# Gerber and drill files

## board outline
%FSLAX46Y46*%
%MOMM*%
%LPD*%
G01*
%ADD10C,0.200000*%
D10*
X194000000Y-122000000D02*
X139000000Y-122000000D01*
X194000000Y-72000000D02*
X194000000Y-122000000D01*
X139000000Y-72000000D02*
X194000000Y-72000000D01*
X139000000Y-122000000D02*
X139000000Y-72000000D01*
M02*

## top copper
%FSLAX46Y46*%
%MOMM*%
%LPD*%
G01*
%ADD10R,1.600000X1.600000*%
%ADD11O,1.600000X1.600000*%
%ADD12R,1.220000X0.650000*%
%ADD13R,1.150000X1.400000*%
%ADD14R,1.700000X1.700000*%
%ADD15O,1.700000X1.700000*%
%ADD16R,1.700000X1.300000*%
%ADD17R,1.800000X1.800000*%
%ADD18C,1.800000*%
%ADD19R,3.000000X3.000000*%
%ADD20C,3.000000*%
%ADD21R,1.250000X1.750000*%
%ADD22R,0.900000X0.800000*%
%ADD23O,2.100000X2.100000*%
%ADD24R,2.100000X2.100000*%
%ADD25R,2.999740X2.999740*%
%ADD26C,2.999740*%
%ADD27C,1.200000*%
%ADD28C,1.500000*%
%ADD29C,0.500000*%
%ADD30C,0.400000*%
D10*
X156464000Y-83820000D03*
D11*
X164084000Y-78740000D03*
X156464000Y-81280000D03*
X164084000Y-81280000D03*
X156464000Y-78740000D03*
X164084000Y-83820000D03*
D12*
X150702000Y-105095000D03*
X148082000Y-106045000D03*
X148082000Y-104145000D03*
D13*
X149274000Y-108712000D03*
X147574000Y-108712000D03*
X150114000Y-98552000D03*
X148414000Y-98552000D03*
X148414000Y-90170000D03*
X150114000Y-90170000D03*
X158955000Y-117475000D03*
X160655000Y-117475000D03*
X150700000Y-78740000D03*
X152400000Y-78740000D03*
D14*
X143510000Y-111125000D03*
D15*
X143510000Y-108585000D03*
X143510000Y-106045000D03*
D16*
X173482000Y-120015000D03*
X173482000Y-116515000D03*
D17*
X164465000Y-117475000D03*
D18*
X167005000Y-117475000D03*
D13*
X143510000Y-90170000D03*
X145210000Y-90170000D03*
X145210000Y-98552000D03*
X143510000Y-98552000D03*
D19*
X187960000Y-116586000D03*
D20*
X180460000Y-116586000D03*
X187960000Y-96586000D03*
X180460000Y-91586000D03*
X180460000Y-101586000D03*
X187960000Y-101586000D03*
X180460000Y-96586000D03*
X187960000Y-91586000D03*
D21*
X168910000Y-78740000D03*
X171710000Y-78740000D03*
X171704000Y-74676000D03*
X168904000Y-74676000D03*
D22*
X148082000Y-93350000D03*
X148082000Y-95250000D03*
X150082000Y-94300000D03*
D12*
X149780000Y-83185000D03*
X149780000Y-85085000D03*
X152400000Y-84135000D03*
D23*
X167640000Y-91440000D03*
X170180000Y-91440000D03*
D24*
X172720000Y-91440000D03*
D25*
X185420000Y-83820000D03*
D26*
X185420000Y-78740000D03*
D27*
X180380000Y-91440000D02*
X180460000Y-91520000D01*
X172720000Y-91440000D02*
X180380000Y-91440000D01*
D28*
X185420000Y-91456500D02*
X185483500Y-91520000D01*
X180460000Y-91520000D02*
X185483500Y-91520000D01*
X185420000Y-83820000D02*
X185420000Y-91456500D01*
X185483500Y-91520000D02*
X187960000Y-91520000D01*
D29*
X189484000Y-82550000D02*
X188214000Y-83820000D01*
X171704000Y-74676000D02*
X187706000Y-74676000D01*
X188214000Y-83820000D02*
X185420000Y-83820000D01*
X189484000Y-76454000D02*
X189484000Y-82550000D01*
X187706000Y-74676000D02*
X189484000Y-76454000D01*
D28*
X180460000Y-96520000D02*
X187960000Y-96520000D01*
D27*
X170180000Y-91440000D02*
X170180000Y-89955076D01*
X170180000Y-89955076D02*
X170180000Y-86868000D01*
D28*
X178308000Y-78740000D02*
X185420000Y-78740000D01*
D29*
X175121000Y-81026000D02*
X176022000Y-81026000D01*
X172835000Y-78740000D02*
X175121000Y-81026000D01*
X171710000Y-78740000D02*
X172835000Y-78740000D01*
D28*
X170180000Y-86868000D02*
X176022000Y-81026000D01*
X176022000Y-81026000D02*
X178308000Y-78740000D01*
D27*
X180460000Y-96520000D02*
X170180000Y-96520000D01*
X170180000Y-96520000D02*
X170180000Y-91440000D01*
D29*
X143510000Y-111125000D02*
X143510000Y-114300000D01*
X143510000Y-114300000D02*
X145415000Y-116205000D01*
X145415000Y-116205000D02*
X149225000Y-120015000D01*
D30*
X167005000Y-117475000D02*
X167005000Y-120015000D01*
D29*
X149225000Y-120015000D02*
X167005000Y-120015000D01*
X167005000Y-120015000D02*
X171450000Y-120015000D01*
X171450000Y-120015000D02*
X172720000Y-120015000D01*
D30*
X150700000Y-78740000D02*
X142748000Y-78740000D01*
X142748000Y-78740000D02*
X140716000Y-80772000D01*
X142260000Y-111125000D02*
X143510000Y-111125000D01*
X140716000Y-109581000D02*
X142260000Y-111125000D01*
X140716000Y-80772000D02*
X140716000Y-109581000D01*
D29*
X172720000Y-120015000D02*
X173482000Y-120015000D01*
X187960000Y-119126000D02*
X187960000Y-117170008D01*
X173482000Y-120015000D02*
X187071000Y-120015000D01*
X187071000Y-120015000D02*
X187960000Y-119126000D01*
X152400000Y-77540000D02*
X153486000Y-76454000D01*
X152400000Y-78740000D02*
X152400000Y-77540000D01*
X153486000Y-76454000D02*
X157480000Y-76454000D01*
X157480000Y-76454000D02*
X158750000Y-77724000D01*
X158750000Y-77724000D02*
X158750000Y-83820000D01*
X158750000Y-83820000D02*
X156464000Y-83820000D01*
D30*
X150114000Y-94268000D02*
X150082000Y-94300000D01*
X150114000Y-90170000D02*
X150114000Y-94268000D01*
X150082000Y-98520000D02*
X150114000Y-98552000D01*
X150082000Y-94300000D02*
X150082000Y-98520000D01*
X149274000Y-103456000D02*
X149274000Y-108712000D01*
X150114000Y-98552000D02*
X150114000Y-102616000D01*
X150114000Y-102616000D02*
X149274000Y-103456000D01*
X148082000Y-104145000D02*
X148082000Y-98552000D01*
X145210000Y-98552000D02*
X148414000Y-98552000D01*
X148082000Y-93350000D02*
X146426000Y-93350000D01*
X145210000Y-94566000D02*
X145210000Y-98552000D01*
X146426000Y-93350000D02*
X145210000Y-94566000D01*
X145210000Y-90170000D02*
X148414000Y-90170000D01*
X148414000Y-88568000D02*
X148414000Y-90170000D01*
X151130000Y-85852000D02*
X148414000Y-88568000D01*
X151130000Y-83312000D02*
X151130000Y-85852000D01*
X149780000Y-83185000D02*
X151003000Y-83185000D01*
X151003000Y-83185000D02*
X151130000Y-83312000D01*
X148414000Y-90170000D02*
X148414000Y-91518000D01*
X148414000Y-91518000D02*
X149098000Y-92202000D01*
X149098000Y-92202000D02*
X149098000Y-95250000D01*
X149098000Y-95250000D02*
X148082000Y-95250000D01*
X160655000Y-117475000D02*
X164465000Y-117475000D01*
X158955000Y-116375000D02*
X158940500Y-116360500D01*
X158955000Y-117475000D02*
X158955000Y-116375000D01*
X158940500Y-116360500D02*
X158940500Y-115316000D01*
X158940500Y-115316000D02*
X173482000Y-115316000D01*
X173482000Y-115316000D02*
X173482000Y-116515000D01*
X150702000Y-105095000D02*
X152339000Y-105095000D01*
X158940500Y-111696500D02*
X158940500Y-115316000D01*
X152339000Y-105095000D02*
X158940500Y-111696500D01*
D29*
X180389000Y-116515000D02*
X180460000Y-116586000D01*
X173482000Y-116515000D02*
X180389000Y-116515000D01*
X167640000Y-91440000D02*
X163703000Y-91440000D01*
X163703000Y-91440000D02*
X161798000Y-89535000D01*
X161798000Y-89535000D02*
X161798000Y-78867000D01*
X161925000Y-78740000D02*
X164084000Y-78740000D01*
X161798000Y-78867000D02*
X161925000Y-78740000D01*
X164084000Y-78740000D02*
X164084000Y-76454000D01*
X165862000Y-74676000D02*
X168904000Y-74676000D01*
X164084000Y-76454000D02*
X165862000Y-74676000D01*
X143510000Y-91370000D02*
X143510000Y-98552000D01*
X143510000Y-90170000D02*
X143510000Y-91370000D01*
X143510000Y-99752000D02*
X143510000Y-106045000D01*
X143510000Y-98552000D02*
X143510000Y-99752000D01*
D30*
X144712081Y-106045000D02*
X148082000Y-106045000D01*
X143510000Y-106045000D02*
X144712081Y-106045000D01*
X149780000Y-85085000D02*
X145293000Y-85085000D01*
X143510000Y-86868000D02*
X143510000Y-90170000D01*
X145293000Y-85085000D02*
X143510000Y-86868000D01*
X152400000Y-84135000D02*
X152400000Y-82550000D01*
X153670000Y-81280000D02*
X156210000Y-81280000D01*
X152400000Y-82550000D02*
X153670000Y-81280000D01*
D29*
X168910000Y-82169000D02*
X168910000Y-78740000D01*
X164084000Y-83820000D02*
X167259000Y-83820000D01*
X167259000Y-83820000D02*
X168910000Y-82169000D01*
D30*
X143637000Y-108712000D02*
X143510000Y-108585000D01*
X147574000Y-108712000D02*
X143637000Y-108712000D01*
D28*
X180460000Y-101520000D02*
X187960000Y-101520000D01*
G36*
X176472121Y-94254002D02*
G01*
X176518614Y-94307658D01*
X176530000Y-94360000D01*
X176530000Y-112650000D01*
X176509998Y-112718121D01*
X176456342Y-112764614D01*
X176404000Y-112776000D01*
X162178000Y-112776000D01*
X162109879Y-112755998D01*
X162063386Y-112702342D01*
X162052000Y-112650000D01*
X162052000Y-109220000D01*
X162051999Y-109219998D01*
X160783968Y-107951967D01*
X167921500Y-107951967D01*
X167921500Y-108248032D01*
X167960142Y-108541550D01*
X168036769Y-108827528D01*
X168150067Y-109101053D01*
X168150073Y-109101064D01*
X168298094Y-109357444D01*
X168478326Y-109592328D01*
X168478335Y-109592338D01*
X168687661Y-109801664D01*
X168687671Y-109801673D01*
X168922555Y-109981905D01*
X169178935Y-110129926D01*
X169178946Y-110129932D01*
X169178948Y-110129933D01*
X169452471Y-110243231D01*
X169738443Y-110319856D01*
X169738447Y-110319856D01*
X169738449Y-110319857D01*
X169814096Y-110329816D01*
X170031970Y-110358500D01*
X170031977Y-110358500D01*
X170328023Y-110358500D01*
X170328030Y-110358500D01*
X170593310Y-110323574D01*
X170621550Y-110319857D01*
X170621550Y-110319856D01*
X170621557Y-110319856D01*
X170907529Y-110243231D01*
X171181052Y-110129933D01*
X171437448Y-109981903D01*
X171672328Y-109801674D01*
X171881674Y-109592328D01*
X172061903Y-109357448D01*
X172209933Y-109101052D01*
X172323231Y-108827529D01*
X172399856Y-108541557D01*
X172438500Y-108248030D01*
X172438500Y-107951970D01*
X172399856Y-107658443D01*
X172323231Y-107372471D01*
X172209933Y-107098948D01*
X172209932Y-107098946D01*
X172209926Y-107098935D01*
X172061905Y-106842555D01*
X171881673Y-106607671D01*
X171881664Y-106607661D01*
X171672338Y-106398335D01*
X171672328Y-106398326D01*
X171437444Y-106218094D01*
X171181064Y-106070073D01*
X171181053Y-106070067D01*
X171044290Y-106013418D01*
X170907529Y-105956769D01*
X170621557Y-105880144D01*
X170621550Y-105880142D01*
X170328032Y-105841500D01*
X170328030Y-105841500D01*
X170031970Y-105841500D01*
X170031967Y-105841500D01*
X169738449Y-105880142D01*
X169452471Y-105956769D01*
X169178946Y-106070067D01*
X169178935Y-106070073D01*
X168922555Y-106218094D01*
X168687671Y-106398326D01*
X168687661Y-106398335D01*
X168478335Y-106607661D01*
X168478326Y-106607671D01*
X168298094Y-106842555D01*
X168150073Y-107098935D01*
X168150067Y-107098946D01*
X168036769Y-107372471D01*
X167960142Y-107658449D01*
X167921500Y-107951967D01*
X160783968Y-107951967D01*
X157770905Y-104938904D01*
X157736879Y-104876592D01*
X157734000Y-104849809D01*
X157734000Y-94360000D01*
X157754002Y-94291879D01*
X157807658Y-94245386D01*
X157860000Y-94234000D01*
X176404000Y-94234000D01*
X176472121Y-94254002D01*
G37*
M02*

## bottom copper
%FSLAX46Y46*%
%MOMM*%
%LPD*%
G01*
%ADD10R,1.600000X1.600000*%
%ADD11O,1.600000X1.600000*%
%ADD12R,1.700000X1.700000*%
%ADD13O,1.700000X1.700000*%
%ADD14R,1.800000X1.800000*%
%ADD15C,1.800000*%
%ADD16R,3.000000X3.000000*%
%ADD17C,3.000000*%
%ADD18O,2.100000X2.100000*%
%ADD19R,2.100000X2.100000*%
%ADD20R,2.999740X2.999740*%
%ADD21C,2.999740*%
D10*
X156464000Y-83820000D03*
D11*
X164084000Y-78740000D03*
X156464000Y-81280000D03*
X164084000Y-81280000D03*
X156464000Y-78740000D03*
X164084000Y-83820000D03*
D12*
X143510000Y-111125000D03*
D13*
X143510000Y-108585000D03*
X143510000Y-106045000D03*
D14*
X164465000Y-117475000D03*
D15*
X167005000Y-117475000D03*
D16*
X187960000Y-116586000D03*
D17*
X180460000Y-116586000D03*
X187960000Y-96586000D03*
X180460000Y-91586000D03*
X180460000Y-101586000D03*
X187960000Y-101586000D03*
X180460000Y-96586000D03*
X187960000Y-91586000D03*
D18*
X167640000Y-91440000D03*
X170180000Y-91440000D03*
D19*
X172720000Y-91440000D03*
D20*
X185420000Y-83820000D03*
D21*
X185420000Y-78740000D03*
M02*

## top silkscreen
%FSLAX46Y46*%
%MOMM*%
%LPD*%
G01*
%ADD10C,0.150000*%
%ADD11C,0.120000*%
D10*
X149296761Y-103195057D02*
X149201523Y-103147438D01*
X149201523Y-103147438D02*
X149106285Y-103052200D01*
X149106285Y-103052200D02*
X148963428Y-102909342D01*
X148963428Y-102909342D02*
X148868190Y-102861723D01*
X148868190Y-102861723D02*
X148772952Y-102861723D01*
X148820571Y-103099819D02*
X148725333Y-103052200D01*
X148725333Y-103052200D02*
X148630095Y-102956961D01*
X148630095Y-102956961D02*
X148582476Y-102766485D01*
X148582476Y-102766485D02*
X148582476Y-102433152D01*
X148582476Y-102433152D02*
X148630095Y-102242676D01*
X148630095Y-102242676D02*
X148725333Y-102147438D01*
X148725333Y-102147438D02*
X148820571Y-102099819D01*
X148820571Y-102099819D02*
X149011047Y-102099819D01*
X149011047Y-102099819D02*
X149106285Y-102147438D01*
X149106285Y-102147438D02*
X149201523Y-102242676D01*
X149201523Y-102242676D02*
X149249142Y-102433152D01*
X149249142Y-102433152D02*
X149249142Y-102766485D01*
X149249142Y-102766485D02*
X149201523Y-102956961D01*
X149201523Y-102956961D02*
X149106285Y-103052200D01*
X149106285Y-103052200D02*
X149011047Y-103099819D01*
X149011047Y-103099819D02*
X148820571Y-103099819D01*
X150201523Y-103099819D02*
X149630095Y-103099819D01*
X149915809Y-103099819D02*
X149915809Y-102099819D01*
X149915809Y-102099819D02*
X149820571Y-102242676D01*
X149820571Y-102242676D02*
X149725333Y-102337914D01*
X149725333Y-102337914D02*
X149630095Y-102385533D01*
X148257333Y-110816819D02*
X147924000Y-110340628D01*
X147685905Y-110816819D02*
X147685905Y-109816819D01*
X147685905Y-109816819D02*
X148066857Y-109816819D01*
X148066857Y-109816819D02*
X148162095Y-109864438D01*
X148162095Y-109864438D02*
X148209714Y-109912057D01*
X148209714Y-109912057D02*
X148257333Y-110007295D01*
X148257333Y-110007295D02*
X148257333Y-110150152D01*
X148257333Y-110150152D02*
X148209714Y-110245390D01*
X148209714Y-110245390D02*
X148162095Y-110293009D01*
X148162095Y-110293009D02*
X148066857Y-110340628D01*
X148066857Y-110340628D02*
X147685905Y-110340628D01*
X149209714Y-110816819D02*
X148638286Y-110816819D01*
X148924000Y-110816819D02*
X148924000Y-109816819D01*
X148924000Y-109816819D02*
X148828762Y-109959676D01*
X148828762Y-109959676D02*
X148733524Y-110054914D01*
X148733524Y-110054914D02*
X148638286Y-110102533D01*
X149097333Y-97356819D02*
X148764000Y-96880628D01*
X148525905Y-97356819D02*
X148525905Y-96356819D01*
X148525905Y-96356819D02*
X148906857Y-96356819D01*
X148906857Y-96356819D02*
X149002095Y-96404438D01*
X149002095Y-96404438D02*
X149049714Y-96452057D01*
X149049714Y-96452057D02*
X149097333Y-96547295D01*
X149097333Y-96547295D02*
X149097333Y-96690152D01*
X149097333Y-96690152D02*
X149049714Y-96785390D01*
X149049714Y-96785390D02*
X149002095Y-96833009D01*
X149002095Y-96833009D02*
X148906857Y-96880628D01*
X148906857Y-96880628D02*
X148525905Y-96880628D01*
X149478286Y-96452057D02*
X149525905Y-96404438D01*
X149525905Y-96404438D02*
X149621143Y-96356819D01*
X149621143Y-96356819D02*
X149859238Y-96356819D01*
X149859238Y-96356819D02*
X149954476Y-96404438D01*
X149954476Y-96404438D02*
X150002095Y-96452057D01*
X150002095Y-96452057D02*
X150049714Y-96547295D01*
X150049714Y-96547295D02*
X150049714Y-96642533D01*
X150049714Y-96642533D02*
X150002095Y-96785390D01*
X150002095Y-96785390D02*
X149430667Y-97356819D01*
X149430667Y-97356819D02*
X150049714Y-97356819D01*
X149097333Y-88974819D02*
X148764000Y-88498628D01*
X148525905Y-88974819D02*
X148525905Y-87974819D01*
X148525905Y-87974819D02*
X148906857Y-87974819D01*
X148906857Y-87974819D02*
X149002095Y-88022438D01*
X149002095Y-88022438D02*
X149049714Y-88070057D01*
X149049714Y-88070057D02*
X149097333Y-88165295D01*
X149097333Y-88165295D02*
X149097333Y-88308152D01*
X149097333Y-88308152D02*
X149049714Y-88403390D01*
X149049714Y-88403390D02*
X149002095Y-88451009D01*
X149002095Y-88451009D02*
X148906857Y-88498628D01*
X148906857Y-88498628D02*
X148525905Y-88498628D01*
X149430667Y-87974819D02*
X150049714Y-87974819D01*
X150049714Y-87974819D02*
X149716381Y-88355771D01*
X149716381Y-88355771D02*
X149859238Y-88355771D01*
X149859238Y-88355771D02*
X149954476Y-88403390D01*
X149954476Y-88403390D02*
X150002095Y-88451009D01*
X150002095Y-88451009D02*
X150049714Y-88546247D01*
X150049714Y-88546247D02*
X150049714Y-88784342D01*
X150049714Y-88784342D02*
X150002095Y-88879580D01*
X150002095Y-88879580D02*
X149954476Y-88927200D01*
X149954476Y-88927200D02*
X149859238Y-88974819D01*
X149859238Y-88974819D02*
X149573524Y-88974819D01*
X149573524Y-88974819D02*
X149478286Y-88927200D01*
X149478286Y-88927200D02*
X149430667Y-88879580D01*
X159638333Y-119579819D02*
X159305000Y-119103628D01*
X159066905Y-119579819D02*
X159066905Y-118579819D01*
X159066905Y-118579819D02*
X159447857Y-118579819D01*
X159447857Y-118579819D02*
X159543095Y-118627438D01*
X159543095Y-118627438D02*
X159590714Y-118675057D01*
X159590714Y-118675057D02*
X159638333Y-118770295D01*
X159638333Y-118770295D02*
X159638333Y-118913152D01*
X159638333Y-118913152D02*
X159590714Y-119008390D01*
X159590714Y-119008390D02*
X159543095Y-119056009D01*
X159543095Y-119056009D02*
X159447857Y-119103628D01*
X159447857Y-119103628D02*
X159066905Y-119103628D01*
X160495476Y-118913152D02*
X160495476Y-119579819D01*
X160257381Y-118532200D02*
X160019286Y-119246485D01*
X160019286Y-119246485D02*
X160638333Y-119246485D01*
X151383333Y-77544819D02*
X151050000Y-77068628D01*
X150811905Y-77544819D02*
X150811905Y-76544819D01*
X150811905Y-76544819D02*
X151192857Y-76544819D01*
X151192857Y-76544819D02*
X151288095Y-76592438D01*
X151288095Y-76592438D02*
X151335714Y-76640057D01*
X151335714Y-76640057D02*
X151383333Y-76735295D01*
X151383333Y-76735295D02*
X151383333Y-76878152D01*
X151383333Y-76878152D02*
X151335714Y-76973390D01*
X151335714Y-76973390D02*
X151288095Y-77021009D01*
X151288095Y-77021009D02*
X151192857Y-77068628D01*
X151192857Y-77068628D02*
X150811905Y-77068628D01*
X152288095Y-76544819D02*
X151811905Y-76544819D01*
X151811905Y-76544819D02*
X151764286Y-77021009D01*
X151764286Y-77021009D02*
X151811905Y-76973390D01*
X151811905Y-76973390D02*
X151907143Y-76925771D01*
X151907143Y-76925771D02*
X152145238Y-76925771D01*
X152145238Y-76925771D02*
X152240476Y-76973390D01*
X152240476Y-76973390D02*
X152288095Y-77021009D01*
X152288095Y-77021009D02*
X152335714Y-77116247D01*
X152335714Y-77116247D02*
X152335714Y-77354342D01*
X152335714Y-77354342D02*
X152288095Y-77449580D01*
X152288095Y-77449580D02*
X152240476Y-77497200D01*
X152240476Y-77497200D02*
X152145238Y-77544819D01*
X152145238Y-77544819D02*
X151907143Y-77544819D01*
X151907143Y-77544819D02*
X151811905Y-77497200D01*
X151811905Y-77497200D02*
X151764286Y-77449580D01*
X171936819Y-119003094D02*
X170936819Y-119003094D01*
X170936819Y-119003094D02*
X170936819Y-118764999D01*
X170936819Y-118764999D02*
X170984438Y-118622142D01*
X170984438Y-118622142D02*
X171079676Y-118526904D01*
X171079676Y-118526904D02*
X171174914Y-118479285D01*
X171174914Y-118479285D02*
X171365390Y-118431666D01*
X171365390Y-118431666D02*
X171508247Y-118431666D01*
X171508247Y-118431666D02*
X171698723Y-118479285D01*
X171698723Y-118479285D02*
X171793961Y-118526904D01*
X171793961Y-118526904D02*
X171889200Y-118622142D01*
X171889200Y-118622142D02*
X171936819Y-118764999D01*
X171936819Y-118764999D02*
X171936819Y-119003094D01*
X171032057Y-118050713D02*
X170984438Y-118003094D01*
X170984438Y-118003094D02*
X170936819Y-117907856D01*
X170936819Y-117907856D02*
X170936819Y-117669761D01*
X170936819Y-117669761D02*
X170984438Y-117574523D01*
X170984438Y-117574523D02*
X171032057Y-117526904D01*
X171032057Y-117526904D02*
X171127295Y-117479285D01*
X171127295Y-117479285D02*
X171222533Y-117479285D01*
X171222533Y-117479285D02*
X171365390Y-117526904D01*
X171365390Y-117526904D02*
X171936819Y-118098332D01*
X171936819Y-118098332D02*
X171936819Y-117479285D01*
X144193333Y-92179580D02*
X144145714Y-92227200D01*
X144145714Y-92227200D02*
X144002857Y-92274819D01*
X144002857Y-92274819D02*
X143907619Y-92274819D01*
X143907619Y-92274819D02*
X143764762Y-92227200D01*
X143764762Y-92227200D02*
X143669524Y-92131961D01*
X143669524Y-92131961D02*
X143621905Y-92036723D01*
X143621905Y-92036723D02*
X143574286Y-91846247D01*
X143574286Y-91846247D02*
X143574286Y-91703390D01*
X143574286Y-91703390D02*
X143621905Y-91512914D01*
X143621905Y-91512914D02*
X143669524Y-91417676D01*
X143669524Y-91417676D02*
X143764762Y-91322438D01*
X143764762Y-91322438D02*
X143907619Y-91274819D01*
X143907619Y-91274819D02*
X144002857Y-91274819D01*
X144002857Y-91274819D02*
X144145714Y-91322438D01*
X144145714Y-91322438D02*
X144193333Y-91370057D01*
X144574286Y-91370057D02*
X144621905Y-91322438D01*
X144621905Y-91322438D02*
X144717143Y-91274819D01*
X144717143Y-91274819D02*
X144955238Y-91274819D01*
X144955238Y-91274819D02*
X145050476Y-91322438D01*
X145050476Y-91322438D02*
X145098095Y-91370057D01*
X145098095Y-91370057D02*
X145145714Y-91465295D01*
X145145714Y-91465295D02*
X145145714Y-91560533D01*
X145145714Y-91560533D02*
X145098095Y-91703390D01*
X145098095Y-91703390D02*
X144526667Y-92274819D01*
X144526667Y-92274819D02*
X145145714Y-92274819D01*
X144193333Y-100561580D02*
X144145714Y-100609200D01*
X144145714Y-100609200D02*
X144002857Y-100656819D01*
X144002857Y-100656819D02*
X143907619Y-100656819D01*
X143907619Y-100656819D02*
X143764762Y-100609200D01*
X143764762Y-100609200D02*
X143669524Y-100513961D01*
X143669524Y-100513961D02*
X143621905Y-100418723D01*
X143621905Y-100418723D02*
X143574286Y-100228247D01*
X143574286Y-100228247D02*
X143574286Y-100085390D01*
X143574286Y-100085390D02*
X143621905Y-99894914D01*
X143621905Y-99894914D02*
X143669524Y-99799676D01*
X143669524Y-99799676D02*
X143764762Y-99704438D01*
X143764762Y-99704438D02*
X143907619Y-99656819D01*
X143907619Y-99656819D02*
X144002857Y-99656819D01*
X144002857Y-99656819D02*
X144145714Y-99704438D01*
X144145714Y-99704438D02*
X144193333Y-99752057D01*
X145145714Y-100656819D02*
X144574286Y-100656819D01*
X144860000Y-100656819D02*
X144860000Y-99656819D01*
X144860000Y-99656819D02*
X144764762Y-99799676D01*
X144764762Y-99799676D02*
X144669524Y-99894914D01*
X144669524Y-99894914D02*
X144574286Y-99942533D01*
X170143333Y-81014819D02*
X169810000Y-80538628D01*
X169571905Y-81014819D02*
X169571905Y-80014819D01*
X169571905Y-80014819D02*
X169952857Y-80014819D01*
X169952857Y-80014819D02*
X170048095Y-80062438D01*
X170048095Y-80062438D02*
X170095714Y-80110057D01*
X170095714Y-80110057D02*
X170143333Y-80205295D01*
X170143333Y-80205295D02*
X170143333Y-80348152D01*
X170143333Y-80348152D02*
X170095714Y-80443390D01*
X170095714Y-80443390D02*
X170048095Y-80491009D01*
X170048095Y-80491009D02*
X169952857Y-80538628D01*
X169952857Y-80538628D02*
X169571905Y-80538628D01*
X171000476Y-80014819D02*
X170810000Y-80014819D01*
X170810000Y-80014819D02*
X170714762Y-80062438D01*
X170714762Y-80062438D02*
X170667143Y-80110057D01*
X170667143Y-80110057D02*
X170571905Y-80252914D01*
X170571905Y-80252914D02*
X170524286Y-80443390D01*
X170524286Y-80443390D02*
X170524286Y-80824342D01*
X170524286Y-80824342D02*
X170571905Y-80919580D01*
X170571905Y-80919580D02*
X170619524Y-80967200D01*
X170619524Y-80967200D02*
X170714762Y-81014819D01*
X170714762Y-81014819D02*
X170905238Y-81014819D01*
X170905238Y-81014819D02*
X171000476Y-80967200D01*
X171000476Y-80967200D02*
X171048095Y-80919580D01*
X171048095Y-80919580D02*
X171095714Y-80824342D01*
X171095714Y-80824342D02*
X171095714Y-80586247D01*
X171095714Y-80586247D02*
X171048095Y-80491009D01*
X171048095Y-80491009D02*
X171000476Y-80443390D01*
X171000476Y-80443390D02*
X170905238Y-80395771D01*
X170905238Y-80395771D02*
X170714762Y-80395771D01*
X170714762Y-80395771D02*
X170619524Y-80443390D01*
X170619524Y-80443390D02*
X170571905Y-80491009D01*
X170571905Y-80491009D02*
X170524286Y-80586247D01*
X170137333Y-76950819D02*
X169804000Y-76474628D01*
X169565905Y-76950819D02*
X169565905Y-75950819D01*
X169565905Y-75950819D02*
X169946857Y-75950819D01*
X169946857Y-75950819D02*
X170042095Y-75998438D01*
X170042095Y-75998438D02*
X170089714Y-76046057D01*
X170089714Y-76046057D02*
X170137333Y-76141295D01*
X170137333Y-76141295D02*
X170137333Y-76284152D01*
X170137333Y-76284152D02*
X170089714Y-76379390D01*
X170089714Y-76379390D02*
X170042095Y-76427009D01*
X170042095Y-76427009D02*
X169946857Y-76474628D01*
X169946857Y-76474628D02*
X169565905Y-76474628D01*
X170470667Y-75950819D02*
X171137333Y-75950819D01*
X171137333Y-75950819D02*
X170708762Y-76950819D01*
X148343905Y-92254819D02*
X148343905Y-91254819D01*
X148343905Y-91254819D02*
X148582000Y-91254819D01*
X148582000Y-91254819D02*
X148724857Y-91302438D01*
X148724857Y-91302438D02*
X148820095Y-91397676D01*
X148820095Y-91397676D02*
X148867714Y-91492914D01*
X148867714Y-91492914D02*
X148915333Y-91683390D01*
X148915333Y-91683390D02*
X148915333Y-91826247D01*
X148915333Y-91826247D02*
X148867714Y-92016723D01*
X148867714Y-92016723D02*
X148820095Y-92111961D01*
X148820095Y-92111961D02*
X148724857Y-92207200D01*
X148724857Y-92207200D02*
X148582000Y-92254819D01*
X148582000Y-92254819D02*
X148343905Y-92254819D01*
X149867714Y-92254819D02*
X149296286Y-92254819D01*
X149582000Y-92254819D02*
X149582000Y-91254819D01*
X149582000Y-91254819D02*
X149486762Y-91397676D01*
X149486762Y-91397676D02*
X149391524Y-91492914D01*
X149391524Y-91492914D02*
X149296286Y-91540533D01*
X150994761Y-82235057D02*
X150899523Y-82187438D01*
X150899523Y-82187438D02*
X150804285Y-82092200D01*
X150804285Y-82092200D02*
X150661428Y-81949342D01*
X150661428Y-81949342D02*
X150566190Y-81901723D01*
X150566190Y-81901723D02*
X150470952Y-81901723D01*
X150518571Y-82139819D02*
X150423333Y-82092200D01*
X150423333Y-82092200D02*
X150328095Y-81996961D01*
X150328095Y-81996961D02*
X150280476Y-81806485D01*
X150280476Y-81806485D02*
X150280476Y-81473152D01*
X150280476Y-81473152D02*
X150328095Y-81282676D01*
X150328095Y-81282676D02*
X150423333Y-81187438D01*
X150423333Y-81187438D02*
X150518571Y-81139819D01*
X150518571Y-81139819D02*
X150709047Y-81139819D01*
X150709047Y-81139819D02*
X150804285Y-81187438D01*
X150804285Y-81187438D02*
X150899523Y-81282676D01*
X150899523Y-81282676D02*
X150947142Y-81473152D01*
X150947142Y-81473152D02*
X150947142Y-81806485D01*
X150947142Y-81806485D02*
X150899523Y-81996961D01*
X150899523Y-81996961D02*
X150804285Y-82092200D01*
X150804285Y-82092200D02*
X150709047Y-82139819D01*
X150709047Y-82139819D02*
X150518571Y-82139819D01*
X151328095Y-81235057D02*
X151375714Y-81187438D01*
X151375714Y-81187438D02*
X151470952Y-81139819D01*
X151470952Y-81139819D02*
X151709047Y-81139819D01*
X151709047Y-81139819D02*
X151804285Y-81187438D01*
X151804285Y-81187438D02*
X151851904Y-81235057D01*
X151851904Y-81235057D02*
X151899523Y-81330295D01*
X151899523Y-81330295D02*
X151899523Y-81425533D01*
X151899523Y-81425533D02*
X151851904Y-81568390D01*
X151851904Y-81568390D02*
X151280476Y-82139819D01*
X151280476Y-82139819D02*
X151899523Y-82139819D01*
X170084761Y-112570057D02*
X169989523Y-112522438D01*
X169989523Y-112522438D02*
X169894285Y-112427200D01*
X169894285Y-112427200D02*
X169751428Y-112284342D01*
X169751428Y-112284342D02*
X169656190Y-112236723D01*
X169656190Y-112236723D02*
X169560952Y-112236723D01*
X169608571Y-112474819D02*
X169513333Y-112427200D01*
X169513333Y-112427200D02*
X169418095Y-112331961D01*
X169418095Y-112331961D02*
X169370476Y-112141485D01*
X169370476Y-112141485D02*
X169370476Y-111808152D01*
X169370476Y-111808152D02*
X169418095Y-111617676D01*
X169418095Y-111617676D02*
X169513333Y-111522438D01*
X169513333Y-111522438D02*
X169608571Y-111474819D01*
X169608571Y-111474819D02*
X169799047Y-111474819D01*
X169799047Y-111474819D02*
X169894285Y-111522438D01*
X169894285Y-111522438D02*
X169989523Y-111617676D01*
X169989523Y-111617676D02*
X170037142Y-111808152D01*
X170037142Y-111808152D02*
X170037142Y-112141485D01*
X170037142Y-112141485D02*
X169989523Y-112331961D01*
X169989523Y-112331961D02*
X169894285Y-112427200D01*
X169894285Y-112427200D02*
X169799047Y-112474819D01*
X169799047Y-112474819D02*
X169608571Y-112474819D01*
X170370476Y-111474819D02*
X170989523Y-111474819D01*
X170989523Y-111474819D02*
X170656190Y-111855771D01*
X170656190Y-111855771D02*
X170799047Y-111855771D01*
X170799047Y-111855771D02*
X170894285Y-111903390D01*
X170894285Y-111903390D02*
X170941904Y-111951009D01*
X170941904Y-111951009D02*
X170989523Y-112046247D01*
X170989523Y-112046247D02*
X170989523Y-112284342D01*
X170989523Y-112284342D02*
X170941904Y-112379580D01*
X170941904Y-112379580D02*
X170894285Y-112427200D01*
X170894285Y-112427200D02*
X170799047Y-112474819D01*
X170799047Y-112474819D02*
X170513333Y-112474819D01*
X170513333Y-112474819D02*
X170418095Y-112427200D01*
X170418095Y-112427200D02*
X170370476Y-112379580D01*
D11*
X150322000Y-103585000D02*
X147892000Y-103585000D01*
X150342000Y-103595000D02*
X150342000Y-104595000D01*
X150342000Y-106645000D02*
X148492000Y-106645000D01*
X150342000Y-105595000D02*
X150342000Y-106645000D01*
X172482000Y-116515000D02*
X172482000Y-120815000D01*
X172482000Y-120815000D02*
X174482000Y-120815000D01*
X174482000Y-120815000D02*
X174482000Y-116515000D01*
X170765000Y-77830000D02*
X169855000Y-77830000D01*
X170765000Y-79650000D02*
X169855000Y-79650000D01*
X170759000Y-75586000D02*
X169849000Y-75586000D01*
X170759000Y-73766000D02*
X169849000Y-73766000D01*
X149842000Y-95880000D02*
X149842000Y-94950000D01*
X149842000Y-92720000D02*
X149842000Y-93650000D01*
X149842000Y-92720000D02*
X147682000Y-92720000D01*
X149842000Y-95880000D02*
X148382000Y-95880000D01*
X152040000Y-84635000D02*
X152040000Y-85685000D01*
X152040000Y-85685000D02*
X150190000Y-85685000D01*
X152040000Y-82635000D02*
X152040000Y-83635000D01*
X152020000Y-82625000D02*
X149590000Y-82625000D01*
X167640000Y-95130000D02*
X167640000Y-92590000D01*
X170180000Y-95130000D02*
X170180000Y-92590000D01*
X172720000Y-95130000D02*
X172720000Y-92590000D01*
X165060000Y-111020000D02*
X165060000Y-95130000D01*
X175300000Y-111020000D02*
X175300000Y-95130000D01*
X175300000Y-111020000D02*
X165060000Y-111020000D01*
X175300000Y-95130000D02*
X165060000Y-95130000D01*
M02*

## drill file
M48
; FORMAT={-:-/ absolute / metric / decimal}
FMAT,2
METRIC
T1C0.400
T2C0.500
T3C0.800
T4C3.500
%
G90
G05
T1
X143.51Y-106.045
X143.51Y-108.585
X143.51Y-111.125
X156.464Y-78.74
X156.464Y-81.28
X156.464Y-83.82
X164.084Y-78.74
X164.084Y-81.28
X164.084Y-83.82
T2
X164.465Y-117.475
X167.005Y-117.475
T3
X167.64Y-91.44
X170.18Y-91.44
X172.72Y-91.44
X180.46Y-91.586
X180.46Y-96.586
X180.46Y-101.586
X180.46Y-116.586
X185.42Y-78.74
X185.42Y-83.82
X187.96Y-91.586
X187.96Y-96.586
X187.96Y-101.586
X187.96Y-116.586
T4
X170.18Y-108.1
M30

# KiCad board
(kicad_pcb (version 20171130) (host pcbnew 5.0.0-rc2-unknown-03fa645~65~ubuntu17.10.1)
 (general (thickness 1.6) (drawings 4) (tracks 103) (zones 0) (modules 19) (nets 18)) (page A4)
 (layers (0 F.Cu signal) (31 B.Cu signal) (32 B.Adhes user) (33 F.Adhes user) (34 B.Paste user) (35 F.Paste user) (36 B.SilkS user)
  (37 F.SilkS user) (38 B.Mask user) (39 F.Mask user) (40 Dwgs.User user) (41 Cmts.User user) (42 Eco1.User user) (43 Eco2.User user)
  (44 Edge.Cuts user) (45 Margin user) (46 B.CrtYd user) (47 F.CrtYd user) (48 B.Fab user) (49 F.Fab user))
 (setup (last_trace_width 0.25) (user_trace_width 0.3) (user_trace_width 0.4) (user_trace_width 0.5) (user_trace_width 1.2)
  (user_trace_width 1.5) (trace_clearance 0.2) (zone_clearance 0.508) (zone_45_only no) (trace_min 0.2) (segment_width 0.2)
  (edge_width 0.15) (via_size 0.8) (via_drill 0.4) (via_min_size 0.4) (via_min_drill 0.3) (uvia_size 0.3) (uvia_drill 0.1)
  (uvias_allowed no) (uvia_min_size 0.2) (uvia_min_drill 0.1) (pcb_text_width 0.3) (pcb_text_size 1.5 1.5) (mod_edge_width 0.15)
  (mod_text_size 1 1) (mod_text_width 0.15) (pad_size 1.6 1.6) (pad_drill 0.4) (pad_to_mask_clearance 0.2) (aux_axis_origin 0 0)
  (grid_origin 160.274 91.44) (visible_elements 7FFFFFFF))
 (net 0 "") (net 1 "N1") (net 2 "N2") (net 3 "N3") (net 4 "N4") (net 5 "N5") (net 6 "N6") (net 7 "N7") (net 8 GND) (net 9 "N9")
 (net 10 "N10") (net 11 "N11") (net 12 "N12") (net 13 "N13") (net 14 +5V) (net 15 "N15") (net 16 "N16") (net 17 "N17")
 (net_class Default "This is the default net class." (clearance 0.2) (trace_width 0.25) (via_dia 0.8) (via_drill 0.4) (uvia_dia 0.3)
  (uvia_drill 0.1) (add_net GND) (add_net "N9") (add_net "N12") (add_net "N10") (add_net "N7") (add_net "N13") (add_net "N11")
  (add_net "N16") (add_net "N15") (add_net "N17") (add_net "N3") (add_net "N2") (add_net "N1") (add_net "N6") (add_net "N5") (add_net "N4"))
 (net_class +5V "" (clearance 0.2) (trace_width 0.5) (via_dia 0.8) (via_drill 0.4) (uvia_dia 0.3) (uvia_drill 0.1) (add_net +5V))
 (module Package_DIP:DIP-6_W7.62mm (layer B.Cu) (at 156.464 83.82)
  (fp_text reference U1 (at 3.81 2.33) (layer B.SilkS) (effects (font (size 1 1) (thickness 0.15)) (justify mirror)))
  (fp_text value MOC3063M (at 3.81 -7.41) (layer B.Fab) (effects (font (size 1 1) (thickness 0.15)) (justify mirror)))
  (pad 1 thru_hole rect (at 0 0) (size 1.6 1.6) (drill 0.4) (layers *.Cu *.Mask) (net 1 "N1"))
  (pad 4 thru_hole oval (at 7.62 -5.08) (size 1.6 1.6) (drill 0.4) (layers *.Cu *.Mask) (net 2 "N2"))
  (pad 2 thru_hole oval (at 0 -2.54) (size 1.6 1.6) (drill 0.4) (layers *.Cu *.Mask) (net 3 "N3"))
  (pad 5 thru_hole oval (at 7.62 -2.54) (size 1.6 1.6) (drill 0.4) (layers *.Cu *.Mask) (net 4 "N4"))
  (pad 3 thru_hole oval (at 0 -5.08) (size 1.6 1.6) (drill 0.4) (layers *.Cu *.Mask) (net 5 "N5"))
  (pad 6 thru_hole oval (at 7.62 0) (size 1.6 1.6) (drill 0.4) (layers *.Cu *.Mask) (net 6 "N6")))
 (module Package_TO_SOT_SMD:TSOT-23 (layer F.Cu) (at 149.392 105.095)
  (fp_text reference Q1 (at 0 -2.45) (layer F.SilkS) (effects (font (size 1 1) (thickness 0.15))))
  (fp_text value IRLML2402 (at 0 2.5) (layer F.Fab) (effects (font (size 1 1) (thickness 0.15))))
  (fp_line (start 0.93 -1.51) (end -1.5 -1.51) (layer F.SilkS) (width 0.12))
  (fp_line (start 0.95 -1.5) (end 0.95 -0.5) (layer F.SilkS) (width 0.12))
  (fp_line (start 0.95 1.55) (end -0.9 1.55) (layer F.SilkS) (width 0.12))
  (fp_line (start 0.95 0.5) (end 0.95 1.55) (layer F.SilkS) (width 0.12))
  (pad 3 smd rect (at 1.31 0) (size 1.22 0.65) (layers F.Cu F.Paste F.Mask) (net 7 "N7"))
  (pad 2 smd rect (at -1.31 0.95) (size 1.22 0.65) (layers F.Cu F.Paste F.Mask) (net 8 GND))
  (pad 1 smd rect (at -1.31 -0.95) (size 1.22 0.65) (layers F.Cu F.Paste F.Mask) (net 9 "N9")))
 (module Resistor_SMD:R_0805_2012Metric (layer F.Cu) (at 148.424 108.712 180)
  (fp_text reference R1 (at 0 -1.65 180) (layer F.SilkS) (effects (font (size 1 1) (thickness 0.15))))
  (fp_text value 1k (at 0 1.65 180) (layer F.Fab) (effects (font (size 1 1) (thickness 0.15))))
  (pad 1 smd rect (at -0.85 0 180) (size 1.15 1.4) (layers F.Cu F.Paste F.Mask) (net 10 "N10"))
  (pad 2 smd rect (at 0.85 0 180) (size 1.15 1.4) (layers F.Cu F.Paste F.Mask) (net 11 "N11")))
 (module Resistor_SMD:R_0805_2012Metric (layer F.Cu) (at 149.264 98.552)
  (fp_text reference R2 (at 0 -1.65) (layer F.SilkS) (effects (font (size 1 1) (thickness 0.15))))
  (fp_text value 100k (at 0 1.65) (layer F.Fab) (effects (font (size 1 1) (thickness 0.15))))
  (pad 2 smd rect (at 0.85 0) (size 1.15 1.4) (layers F.Cu F.Paste F.Mask) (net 10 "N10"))
  (pad 1 smd rect (at -0.85 0) (size 1.15 1.4) (layers F.Cu F.Paste F.Mask) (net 9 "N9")))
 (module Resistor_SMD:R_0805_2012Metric (layer F.Cu) (at 149.264 90.17)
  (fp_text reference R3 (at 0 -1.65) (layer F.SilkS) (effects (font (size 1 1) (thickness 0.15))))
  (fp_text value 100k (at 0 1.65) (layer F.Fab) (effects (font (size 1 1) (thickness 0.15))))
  (pad 1 smd rect (at -0.85 0) (size 1.15 1.4) (layers F.Cu F.Paste F.Mask) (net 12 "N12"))
  (pad 2 smd rect (at 0.85 0) (size 1.15 1.4) (layers F.Cu F.Paste F.Mask) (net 10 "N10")))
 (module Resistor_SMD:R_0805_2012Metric (layer F.Cu) (at 159.805 117.475 180)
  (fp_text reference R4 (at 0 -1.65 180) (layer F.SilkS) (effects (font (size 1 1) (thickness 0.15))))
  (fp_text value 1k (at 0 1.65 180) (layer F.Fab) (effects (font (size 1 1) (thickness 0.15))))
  (pad 2 smd rect (at 0.85 0 180) (size 1.15 1.4) (layers F.Cu F.Paste F.Mask) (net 7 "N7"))
  (pad 1 smd rect (at -0.85 0 180) (size 1.15 1.4) (layers F.Cu F.Paste F.Mask) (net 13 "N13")))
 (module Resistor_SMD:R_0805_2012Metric (layer F.Cu) (at 151.55 78.74)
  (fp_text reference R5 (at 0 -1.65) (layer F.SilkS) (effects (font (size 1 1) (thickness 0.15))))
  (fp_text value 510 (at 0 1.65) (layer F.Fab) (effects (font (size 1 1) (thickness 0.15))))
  (pad 1 smd rect (at -0.85 0) (size 1.15 1.4) (layers F.Cu F.Paste F.Mask) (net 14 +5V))
  (pad 2 smd rect (at 0.85 0) (size 1.15 1.4) (layers F.Cu F.Paste F.Mask) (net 1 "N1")))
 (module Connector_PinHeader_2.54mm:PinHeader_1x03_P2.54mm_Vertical (layer B.Cu) (at 143.51 111.125)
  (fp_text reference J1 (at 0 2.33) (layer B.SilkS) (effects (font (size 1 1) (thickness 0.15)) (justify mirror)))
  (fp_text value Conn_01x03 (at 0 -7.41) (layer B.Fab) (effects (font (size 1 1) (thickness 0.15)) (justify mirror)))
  (pad 1 thru_hole rect (at 0 0) (size 1.7 1.7) (drill 0.4) (layers *.Cu *.Mask) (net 14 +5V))
  (pad 2 thru_hole oval (at 0 -2.54) (size 1.7 1.7) (drill 0.4) (layers *.Cu *.Mask) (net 11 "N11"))
  (pad 3 thru_hole oval (at 0 -5.08) (size 1.7 1.7) (drill 0.4) (layers *.Cu *.Mask) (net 8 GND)))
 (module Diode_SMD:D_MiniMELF (layer F.Cu) (at 173.482 118.265 90)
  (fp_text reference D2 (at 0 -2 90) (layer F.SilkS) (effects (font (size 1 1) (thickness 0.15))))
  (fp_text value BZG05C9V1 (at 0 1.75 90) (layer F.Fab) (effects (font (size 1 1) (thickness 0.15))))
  (fp_line (start 1.75 -1) (end -2.55 -1) (layer F.SilkS) (width 0.12))
  (fp_line (start -2.55 -1) (end -2.55 1) (layer F.SilkS) (width 0.12))
  (fp_line (start -2.55 1) (end 1.75 1) (layer F.SilkS) (width 0.12))
  (pad 1 smd rect (at -1.75 0 90) (size 1.3 1.7) (layers F.Cu F.Paste F.Mask) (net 14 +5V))
  (pad 2 smd rect (at 1.75 0 90) (size 1.3 1.7) (layers F.Cu F.Paste F.Mask) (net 7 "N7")))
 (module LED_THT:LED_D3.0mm (layer B.Cu) (at 164.465 117.475)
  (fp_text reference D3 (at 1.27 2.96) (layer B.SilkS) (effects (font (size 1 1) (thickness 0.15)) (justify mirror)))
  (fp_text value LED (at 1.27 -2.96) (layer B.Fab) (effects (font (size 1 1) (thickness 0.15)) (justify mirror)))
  (pad 1 thru_hole rect (at 0 0) (size 1.8 1.8) (drill 0.5) (layers *.Cu *.Mask) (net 13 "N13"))
  (pad 2 thru_hole circle (at 2.54 0) (size 1.8 1.8) (drill 0.5) (layers *.Cu *.Mask) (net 14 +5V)))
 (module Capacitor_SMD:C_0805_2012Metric (layer F.Cu) (at 144.36 90.17 180)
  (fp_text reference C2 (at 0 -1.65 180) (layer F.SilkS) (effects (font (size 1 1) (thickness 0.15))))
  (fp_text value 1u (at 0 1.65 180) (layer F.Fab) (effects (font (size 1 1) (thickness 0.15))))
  (pad 2 smd rect (at 0.85 0 180) (size 1.15 1.4) (layers F.Cu F.Paste F.Mask) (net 8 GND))
  (pad 1 smd rect (at -0.85 0 180) (size 1.15 1.4) (layers F.Cu F.Paste F.Mask) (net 12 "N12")))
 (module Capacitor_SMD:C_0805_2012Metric (layer F.Cu) (at 144.36 98.552 180)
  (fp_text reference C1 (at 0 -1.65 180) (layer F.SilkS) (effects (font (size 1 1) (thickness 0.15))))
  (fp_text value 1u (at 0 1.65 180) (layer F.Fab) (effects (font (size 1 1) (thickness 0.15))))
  (pad 1 smd rect (at -0.85 0 180) (size 1.15 1.4) (layers F.Cu F.Paste F.Mask) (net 9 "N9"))
  (pad 2 smd rect (at 0.85 0 180) (size 1.15 1.4) (layers F.Cu F.Paste F.Mask) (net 8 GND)))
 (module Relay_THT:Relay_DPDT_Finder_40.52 (layer B.Cu) (at 187.96 116.586 90)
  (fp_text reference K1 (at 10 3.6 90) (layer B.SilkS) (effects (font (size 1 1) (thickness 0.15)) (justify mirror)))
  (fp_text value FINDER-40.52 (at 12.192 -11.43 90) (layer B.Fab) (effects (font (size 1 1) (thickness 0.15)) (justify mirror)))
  (pad A1 thru_hole rect (at 0 0 90) (size 3 3) (drill 0.8) (layers *.Cu *.Mask) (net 14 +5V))
  (pad A2 thru_hole circle (at 0 -7.5 90) (size 3 3) (drill 0.8) (layers *.Cu *.Mask) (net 7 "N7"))
  (pad 11 thru_hole circle (at 20 0 90) (size 3 3) (drill 0.8) (layers *.Cu *.Mask) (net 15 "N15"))
  (pad 24 thru_hole circle (at 25 -7.5 90) (size 3 3) (drill 0.8) (layers *.Cu *.Mask) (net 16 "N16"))
  (pad 22 thru_hole circle (at 15 -7.5 90) (size 3 3) (drill 0.8) (layers *.Cu *.Mask) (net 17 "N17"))
  (pad 12 thru_hole circle (at 15 0 90) (size 3 3) (drill 0.8) (layers *.Cu *.Mask) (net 17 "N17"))
  (pad 21 thru_hole circle (at 20 -7.5 90) (size 3 3) (drill 0.8) (layers *.Cu *.Mask) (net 15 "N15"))
  (pad 14 thru_hole circle (at 25 0 90) (size 3 3) (drill 0.8) (layers *.Cu *.Mask) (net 16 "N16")))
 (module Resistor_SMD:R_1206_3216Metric (layer F.Cu) (at 170.31 78.74 180)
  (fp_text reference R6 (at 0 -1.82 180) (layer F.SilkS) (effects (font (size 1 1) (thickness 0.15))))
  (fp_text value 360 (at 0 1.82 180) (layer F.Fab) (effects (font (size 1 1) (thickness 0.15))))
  (fp_line (start -0.455 0.91) (end 0.455 0.91) (layer F.SilkS) (width 0.12))
  (fp_line (start -0.455 -0.91) (end 0.455 -0.91) (layer F.SilkS) (width 0.12))
  (pad 2 smd rect (at 1.4 0 180) (size 1.25 1.75) (layers F.Cu F.Paste F.Mask) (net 6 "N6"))
  (pad 1 smd rect (at -1.4 0 180) (size 1.25 1.75) (layers F.Cu F.Paste F.Mask) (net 15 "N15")))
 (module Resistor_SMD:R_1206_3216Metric (layer F.Cu) (at 170.304 74.676 180)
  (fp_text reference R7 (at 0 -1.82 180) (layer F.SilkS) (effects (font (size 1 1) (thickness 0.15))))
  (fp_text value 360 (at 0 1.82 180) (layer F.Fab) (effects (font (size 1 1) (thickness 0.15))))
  (fp_line (start -0.455 -0.91) (end 0.455 -0.91) (layer F.SilkS) (width 0.12))
  (fp_line (start -0.455 0.91) (end 0.455 0.91) (layer F.SilkS) (width 0.12))
  (pad 1 smd rect (at -1.4 0 180) (size 1.25 1.75) (layers F.Cu F.Paste F.Mask) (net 16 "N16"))
  (pad 2 smd rect (at 1.4 0 180) (size 1.25 1.75) (layers F.Cu F.Paste F.Mask) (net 2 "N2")))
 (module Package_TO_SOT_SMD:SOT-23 (layer F.Cu) (at 149.082 94.3)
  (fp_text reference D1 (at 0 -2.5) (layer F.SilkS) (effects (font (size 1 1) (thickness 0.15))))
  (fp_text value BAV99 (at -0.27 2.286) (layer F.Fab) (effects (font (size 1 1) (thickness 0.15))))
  (fp_line (start 0.76 1.58) (end 0.76 0.65) (layer F.SilkS) (width 0.12))
  (fp_line (start 0.76 -1.58) (end 0.76 -0.65) (layer F.SilkS) (width 0.12))
  (fp_line (start 0.76 -1.58) (end -1.4 -1.58) (layer F.SilkS) (width 0.12))
  (fp_line (start 0.76 1.58) (end -0.7 1.58) (layer F.SilkS) (width 0.12))
  (pad 1 smd rect (at -1 -0.95) (size 0.9 0.8) (layers F.Cu F.Paste F.Mask) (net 9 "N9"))
  (pad 2 smd rect (at -1 0.95) (size 0.9 0.8) (layers F.Cu F.Paste F.Mask) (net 12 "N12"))
  (pad 3 smd rect (at 1 0) (size 0.9 0.8) (layers F.Cu F.Paste F.Mask) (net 10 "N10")))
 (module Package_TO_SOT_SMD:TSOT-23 (layer F.Cu) (at 151.09 84.135)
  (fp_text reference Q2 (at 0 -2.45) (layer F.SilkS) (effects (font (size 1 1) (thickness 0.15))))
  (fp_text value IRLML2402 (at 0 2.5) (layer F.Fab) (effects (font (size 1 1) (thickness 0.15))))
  (fp_line (start 0.95 0.5) (end 0.95 1.55) (layer F.SilkS) (width 0.12))
  (fp_line (start 0.95 1.55) (end -0.9 1.55) (layer F.SilkS) (width 0.12))
  (fp_line (start 0.95 -1.5) (end 0.95 -0.5) (layer F.SilkS) (width 0.12))
  (fp_line (start 0.93 -1.51) (end -1.5 -1.51) (layer F.SilkS) (width 0.12))
  (pad 1 smd rect (at -1.31 -0.95) (size 1.22 0.65) (layers F.Cu F.Paste F.Mask) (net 12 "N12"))
  (pad 2 smd rect (at -1.31 0.95) (size 1.22 0.65) (layers F.Cu F.Paste F.Mask) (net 8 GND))
  (pad 3 smd rect (at 1.31 0) (size 1.22 0.65) (layers F.Cu F.Paste F.Mask) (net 3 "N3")))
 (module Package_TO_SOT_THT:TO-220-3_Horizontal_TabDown (layer F.Cu) (at 172.72 91.44 180)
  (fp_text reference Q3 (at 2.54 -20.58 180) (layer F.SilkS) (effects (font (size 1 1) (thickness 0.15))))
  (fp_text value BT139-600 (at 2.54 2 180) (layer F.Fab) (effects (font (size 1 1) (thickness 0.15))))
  (fp_line (start 5.08 -3.69) (end 5.08 -1.15) (layer F.SilkS) (width 0.12))
  (fp_line (start 2.54 -3.69) (end 2.54 -1.15) (layer F.SilkS) (width 0.12))
  (fp_line (start 0 -3.69) (end 0 -1.15) (layer F.SilkS) (width 0.12))
  (fp_line (start 7.66 -19.58) (end 7.66 -3.69) (layer F.SilkS) (width 0.12))
  (fp_line (start -2.58 -19.58) (end -2.58 -3.69) (layer F.SilkS) (width 0.12))
  (fp_line (start -2.58 -19.58) (end 7.66 -19.58) (layer F.SilkS) (width 0.12))
  (fp_line (start -2.58 -3.69) (end 7.66 -3.69) (layer F.SilkS) (width 0.12))
  (pad 3 thru_hole oval (at 5.08 0 180) (size 2.1 2.1) (drill 0.8) (layers *.Cu *.Mask) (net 2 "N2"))
  (pad 2 thru_hole oval (at 2.54 0 180) (size 2.1 2.1) (drill 0.8) (layers *.Cu *.Mask) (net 15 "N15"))
  (pad 1 thru_hole rect (at 0 0 180) (size 2.1 2.1) (drill 0.8) (layers *.Cu *.Mask) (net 16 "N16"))
  (pad "" np_thru_hole oval (at 2.54 -16.66 180) (size 3.5 3.5) (drill 3.5) (layers *.Cu *.Mask)))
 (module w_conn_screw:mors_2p (layer B.Cu) (at 185.42 81.28 90)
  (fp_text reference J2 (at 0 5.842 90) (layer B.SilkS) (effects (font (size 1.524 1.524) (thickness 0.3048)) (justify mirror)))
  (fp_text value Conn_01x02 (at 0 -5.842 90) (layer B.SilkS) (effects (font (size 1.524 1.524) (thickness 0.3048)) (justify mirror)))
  (pad 1 thru_hole rect (at -2.54 0 90) (size 2.99974 2.99974) (drill 0.8) (layers *.Cu *.Mask B.SilkS) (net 16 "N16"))
  (pad 2 thru_hole circle (at 2.54 0 90) (size 2.99974 2.99974) (drill 0.8) (layers *.Cu *.Mask B.SilkS) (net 15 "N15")))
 (gr_line (start 194 122) (end 139 122) (layer Edge.Cuts) (width 0.2))
 (gr_line (start 194 72) (end 194 122) (layer Edge.Cuts) (width 0.2))
 (gr_line (start 139 72) (end 194 72) (layer Edge.Cuts) (width 0.2))
 (gr_line (start 139 122) (end 139 72) (layer Edge.Cuts) (width 0.2))
 (segment (start 180.38 91.44) (end 180.46 91.52) (width 1.2) (layer F.Cu) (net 16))
 (segment (start 172.72 91.44) (end 180.38 91.44) (width 1.2) (layer F.Cu) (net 16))
 (segment (start 185.42 91.4565) (end 185.4835 91.52) (width 1.5) (layer F.Cu) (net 16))
 (segment (start 180.46 91.52) (end 185.4835 91.52) (width 1.5) (layer F.Cu) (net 16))
 (segment (start 185.42 83.82) (end 185.42 91.4565) (width 1.5) (layer F.Cu) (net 16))
 (segment (start 185.4835 91.52) (end 187.96 91.52) (width 1.5) (layer F.Cu) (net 16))
 (segment (start 189.484 82.55) (end 188.214 83.82) (width 0.5) (layer F.Cu) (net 16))
 (segment (start 171.704 74.676) (end 187.706 74.676) (width 0.5) (layer F.Cu) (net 16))
 (segment (start 188.214 83.82) (end 185.42 83.82) (width 0.5) (layer F.Cu) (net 16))
 (segment (start 189.484 76.454) (end 189.484 82.55) (width 0.5) (layer F.Cu) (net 16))
 (segment (start 187.706 74.676) (end 189.484 76.454) (width 0.5) (layer F.Cu) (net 16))
 (segment (start 180.46 96.52) (end 187.96 96.52) (width 1.5) (layer F.Cu) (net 15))
 (segment (start 170.18 91.44) (end 170.18 89.955076) (width 1.2) (layer F.Cu) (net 15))
 (segment (start 170.18 89.955076) (end 170.18 86.868) (width 1.2) (layer F.Cu) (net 15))
 (segment (start 178.308 78.74) (end 185.42 78.74) (width 1.5) (layer F.Cu) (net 15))
 (segment (start 175.121 81.026) (end 176.022 81.026) (width 0.5) (layer F.Cu) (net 15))
 (segment (start 172.835 78.74) (end 175.121 81.026) (width 0.5) (layer F.Cu) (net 15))
 (segment (start 171.71 78.74) (end 172.835 78.74) (width 0.5) (layer F.Cu) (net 15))
 (segment (start 170.18 86.868) (end 176.022 81.026) (width 1.5) (layer F.Cu) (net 15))
 (segment (start 176.022 81.026) (end 178.308 78.74) (width 1.5) (layer F.Cu) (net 15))
 (segment (start 180.46 96.52) (end 170.18 96.52) (width 1.2) (layer F.Cu) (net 15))
 (segment (start 170.18 96.52) (end 170.18 91.44) (width 1.2) (layer F.Cu) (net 15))
 (segment (start 143.51 111.125) (end 143.51 114.3) (width 0.5) (layer F.Cu) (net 14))
 (segment (start 143.51 114.3) (end 145.415 116.205) (width 0.5) (layer F.Cu) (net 14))
 (segment (start 145.415 116.205) (end 149.225 120.015) (width 0.5) (layer F.Cu) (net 14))
 (segment (start 167.005 117.475) (end 167.005 120.015) (width 0.4) (layer F.Cu) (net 14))
 (segment (start 149.225 120.015) (end 167.005 120.015) (width 0.5) (layer F.Cu) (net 14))
 (segment (start 167.005 120.015) (end 171.45 120.015) (width 0.5) (layer F.Cu) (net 14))
 (segment (start 171.45 120.015) (end 172.72 120.015) (width 0.5) (layer F.Cu) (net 14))
 (segment (start 150.7 78.74) (end 142.748 78.74) (width 0.4) (layer F.Cu) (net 14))
 (segment (start 142.748 78.74) (end 140.716 80.772) (width 0.4) (layer F.Cu) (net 14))
 (segment (start 142.26 111.125) (end 143.51 111.125) (width 0.4) (layer F.Cu) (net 14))
 (segment (start 140.716 109.581) (end 142.26 111.125) (width 0.4) (layer F.Cu) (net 14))
 (segment (start 140.716 80.772) (end 140.716 109.581) (width 0.4) (layer F.Cu) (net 14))
 (segment (start 172.72 120.015) (end 173.482 120.015) (width 0.5) (layer F.Cu) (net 14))
 (segment (start 187.96 119.126) (end 187.96 117.170008) (width 0.5) (layer F.Cu) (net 14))
 (segment (start 173.482 120.015) (end 187.071 120.015) (width 0.5) (layer F.Cu) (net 14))
 (segment (start 187.071 120.015) (end 187.96 119.126) (width 0.5) (layer F.Cu) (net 14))
 (segment (start 152.4 77.54) (end 153.486 76.454) (width 0.5) (layer F.Cu) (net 1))
 (segment (start 152.4 78.74) (end 152.4 77.54) (width 0.5) (layer F.Cu) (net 1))
 (segment (start 153.486 76.454) (end 157.48 76.454) (width 0.5) (layer F.Cu) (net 1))
 (segment (start 157.48 76.454) (end 158.75 77.724) (width 0.5) (layer F.Cu) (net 1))
 (segment (start 158.75 77.724) (end 158.75 83.82) (width 0.5) (layer F.Cu) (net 1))
 (segment (start 158.75 83.82) (end 156.464 83.82) (width 0.5) (layer F.Cu) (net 1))
 (segment (start 150.114 94.268) (end 150.082 94.3) (width 0.4) (layer F.Cu) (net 10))
 (segment (start 150.114 90.17) (end 150.114 94.268) (width 0.4) (layer F.Cu) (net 10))
 (segment (start 150.082 98.52) (end 150.114 98.552) (width 0.4) (layer F.Cu) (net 10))
 (segment (start 150.082 94.3) (end 150.082 98.52) (width 0.4) (layer F.Cu) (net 10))
 (segment (start 149.274 103.456) (end 149.274 108.712) (width 0.4) (layer F.Cu) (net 10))
 (segment (start 150.114 98.552) (end 150.114 102.616) (width 0.4) (layer F.Cu) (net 10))
 (segment (start 150.114 102.616) (end 149.274 103.456) (width 0.4) (layer F.Cu) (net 10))
 (segment (start 148.082 104.145) (end 148.082 98.552) (width 0.4) (layer F.Cu) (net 9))
 (segment (start 145.21 98.552) (end 148.414 98.552) (width 0.4) (layer F.Cu) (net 9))
 (segment (start 148.082 93.35) (end 146.426 93.35) (width 0.4) (layer F.Cu) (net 9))
 (segment (start 145.21 94.566) (end 145.21 98.552) (width 0.4) (layer F.Cu) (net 9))
 (segment (start 146.426 93.35) (end 145.21 94.566) (width 0.4) (layer F.Cu) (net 9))
 (segment (start 145.21 90.17) (end 148.414 90.17) (width 0.4) (layer F.Cu) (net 12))
 (segment (start 148.414 88.568) (end 148.414 90.17) (width 0.4) (layer F.Cu) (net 12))
 (segment (start 151.13 85.852) (end 148.414 88.568) (width 0.4) (layer F.Cu) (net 12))
 (segment (start 151.13 83.312) (end 151.13 85.852) (width 0.4) (layer F.Cu) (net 12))
 (segment (start 149.78 83.185) (end 151.003 83.185) (width 0.4) (layer F.Cu) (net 12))
 (segment (start 151.003 83.185) (end 151.13 83.312) (width 0.4) (layer F.Cu) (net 12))
 (segment (start 148.414 90.17) (end 148.414 91.518) (width 0.4) (layer F.Cu) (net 12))
 (segment (start 148.414 91.518) (end 149.098 92.202) (width 0.4) (layer F.Cu) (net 12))
 (segment (start 149.098 92.202) (end 149.098 95.25) (width 0.4) (layer F.Cu) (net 12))
 (segment (start 149.098 95.25) (end 148.082 95.25) (width 0.4) (layer F.Cu) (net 12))
 (segment (start 160.655 117.475) (end 164.465 117.475) (width 0.4) (layer F.Cu) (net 13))
 (segment (start 158.955 116.375) (end 158.9405 116.3605) (width 0.4) (layer F.Cu) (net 7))
 (segment (start 158.955 117.475) (end 158.955 116.375) (width 0.4) (layer F.Cu) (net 7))
 (segment (start 158.9405 116.3605) (end 158.9405 115.316) (width 0.4) (layer F.Cu) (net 7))
 (segment (start 158.9405 115.316) (end 173.482 115.316) (width 0.4) (layer F.Cu) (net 7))
 (segment (start 173.482 115.316) (end 173.482 116.515) (width 0.4) (layer F.Cu) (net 7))
 (segment (start 150.702 105.095) (end 152.339 105.095) (width 0.4) (layer F.Cu) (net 7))
 (segment (start 158.9405 111.6965) (end 158.9405 115.316) (width 0.4) (layer F.Cu) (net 7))
 (segment (start 152.339 105.095) (end 158.9405 111.6965) (width 0.4) (layer F.Cu) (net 7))
 (segment (start 180.389 116.515) (end 180.46 116.586) (width 0.5) (layer F.Cu) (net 7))
 (segment (start 173.482 116.515) (end 180.389 116.515) (width 0.5) (layer F.Cu) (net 7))
 (segment (start 167.64 91.44) (end 163.703 91.44) (width 0.5) (layer F.Cu) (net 2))
 (segment (start 163.703 91.44) (end 161.798 89.535) (width 0.5) (layer F.Cu) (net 2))
 (segment (start 161.798 89.535) (end 161.798 78.867) (width 0.5) (layer F.Cu) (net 2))
 (segment (start 161.925 78.74) (end 164.084 78.74) (width 0.5) (layer F.Cu) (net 2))
 (segment (start 161.798 78.867) (end 161.925 78.74) (width 0.5) (layer F.Cu) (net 2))
 (segment (start 164.084 78.74) (end 164.084 76.454) (width 0.5) (layer F.Cu) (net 2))
 (segment (start 165.862 74.676) (end 168.904 74.676) (width 0.5) (layer F.Cu) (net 2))
 (segment (start 164.084 76.454) (end 165.862 74.676) (width 0.5) (layer F.Cu) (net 2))
 (segment (start 143.51 91.37) (end 143.51 98.552) (width 0.5) (layer F.Cu) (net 8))
 (segment (start 143.51 90.17) (end 143.51 91.37) (width 0.5) (layer F.Cu) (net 8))
 (segment (start 143.51 99.752) (end 143.51 106.045) (width 0.5) (layer F.Cu) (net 8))
 (segment (start 143.51 98.552) (end 143.51 99.752) (width 0.5) (layer F.Cu) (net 8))
 (segment (start 144.712081 106.045) (end 148.082 106.045) (width 0.4) (layer F.Cu) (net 8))
 (segment (start 143.51 106.045) (end 144.712081 106.045) (width 0.4) (layer F.Cu) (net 8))
 (segment (start 149.78 85.085) (end 145.293 85.085) (width 0.4) (layer F.Cu) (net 8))
 (segment (start 143.51 86.868) (end 143.51 90.17) (width 0.4) (layer F.Cu) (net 8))
 (segment (start 145.293 85.085) (end 143.51 86.868) (width 0.4) (layer F.Cu) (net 8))
 (segment (start 152.4 84.135) (end 152.4 82.55) (width 0.4) (layer F.Cu) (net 3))
 (segment (start 153.67 81.28) (end 156.21 81.28) (width 0.4) (layer F.Cu) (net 3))
 (segment (start 152.4 82.55) (end 153.67 81.28) (width 0.4) (layer F.Cu) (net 3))
 (segment (start 168.91 82.169) (end 168.91 78.74) (width 0.5) (layer F.Cu) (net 6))
 (segment (start 164.084 83.82) (end 167.259 83.82) (width 0.5) (layer F.Cu) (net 6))
 (segment (start 167.259 83.82) (end 168.91 82.169) (width 0.5) (layer F.Cu) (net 6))
 (segment (start 143.637 108.712) (end 143.51 108.585) (width 0.4) (layer F.Cu) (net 11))
 (segment (start 147.574 108.712) (end 143.637 108.712) (width 0.4) (layer F.Cu) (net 11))
 (segment (start 180.46 101.52) (end 187.96 101.52) (width 1.5) (layer F.Cu) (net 17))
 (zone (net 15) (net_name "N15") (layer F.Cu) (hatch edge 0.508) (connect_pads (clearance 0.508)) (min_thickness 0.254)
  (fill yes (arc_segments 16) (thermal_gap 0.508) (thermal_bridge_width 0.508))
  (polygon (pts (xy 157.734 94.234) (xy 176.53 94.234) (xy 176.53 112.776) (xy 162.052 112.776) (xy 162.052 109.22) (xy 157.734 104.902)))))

